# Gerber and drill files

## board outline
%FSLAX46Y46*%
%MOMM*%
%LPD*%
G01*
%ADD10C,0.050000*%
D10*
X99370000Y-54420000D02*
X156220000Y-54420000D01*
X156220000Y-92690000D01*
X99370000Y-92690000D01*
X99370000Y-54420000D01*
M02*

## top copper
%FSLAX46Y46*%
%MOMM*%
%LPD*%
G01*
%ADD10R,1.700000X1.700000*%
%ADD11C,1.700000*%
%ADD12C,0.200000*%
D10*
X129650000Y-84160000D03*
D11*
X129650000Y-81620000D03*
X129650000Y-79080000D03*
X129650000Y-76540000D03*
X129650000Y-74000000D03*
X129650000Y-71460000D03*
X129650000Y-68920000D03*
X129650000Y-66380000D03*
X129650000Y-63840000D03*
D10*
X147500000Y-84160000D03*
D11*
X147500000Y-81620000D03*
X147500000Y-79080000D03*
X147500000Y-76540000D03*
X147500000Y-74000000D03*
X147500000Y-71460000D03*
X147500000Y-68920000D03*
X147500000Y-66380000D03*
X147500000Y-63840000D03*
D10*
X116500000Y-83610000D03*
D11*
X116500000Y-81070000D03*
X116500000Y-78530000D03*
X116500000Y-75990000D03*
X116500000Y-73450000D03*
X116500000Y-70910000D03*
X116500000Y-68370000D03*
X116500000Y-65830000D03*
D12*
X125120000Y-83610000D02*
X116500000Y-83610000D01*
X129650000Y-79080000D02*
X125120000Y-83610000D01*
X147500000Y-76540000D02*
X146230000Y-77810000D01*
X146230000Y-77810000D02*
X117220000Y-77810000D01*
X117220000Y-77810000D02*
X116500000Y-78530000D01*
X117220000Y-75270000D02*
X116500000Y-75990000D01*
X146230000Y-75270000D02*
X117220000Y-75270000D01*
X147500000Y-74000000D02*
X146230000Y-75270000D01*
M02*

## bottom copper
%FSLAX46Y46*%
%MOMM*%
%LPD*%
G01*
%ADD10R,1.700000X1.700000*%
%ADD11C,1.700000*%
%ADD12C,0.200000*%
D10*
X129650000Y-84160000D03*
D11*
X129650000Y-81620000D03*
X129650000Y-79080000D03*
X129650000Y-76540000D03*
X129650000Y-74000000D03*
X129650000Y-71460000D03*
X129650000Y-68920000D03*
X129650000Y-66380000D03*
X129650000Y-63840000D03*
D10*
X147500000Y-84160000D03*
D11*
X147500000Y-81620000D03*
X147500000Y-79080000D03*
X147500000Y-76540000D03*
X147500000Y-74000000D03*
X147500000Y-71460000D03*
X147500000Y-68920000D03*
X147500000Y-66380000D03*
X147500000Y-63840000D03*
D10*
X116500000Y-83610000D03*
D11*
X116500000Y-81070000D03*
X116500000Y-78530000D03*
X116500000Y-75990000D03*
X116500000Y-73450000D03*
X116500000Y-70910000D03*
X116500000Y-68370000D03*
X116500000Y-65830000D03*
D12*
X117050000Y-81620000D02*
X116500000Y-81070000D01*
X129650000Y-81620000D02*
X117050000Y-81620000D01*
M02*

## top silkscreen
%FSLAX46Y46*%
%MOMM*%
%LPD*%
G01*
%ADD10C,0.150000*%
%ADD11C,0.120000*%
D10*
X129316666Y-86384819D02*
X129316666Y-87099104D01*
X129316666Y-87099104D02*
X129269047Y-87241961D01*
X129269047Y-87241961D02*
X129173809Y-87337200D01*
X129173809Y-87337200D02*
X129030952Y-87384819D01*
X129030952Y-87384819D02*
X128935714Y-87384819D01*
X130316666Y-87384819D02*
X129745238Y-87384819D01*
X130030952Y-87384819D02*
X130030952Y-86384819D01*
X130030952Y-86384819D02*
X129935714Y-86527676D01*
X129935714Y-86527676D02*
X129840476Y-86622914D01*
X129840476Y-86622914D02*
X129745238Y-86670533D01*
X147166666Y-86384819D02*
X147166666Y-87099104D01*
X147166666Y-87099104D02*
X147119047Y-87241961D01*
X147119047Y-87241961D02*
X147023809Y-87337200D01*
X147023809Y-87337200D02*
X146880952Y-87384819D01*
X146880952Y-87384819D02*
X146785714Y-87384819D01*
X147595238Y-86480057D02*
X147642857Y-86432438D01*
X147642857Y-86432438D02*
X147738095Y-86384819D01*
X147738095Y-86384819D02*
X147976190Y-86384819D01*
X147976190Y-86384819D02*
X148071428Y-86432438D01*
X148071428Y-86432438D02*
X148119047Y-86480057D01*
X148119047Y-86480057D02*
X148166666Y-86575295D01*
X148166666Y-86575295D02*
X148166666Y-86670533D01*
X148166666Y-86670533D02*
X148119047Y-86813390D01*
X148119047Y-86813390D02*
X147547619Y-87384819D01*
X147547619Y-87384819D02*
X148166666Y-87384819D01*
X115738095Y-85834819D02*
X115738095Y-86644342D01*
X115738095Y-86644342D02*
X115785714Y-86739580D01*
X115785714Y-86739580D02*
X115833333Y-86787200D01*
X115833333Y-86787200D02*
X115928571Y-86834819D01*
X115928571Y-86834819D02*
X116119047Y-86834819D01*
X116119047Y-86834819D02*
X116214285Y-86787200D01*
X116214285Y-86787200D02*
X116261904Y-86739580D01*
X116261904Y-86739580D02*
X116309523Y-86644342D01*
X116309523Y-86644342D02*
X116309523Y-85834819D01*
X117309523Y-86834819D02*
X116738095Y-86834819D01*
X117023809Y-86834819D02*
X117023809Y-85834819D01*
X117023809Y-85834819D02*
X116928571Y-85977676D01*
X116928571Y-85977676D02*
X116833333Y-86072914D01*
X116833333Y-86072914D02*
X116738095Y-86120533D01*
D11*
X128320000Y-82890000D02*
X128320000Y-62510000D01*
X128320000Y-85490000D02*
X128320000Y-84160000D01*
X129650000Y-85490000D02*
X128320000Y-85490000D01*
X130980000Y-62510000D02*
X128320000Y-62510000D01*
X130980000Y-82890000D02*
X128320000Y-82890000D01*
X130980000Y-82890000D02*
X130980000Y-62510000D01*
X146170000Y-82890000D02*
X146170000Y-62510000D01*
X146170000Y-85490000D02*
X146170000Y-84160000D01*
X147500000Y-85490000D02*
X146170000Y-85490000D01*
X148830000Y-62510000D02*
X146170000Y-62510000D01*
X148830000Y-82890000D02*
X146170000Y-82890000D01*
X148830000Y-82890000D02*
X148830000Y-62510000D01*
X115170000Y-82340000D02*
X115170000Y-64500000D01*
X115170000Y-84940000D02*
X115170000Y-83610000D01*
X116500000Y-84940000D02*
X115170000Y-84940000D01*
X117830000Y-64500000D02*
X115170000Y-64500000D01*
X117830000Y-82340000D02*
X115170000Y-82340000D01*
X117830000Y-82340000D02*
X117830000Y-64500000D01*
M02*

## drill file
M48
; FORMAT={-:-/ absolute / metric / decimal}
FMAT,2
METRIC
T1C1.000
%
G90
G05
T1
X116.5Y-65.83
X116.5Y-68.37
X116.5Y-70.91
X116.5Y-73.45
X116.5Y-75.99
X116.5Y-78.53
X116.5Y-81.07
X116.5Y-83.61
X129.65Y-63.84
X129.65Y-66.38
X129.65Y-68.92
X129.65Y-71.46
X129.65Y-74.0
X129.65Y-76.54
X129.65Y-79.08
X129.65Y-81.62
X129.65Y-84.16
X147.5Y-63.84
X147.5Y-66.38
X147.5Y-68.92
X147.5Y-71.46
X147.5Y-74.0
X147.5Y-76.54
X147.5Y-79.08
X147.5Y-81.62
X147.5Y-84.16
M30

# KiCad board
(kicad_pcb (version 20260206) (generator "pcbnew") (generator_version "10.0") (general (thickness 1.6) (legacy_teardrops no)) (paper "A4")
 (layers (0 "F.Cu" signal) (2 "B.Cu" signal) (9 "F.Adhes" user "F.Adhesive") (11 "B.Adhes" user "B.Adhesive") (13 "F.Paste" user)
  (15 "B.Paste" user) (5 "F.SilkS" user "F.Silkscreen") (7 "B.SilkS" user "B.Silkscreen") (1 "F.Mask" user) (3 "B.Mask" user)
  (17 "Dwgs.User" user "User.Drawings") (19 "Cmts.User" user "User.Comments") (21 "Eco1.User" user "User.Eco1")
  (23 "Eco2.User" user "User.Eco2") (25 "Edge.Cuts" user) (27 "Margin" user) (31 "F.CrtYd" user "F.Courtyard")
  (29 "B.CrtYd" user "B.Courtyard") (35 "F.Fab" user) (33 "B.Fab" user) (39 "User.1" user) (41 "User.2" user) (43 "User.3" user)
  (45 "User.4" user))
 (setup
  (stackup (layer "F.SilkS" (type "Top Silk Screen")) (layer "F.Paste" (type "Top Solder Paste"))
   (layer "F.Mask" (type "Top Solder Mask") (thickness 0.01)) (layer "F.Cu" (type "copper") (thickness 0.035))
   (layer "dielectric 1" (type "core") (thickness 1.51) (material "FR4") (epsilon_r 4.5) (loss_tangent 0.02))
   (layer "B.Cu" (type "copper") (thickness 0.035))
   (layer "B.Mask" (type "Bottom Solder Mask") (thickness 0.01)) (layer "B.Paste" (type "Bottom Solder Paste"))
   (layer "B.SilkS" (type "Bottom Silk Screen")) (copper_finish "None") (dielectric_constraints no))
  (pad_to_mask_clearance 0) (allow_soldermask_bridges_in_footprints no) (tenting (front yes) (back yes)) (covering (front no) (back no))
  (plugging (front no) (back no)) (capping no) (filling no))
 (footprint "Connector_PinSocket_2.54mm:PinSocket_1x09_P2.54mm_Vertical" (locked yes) (layer "F.Cu") (at 129.65 84.16 180)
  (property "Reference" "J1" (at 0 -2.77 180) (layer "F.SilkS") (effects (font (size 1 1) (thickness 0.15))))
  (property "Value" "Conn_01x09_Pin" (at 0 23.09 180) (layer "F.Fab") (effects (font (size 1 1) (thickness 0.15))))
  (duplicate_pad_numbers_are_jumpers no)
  (fp_line (start 1.33 1.27) (end 1.33 21.65) (stroke (width 0.12) (type solid)) (layer "F.SilkS"))
  (fp_line (start 1.33 -1.33) (end 1.33 0) (stroke (width 0.12) (type solid)) (layer "F.SilkS"))
  (fp_line (start 0 -1.33) (end 1.33 -1.33) (stroke (width 0.12) (type solid)) (layer "F.SilkS"))
  (fp_line (start -1.33 21.65) (end 1.33 21.65) (stroke (width 0.12) (type solid)) (layer "F.SilkS"))
  (fp_line (start -1.33 1.27) (end 1.33 1.27) (stroke (width 0.12) (type solid)) (layer "F.SilkS"))
  (fp_line (start -1.33 1.27) (end -1.33 21.65) (stroke (width 0.12) (type solid)) (layer "F.SilkS"))
  (pad "1" thru_hole rect (at 0 0 180) (size 1.7 1.7) (drill 1) (layers "*.Cu" "*.Mask") (remove_unused_layers no)
   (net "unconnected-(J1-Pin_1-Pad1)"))
  (pad "2" thru_hole circle (at 0 2.54 180) (size 1.7 1.7) (drill 1) (layers "*.Cu" "*.Mask") (remove_unused_layers no)
   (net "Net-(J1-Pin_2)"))
  (pad "3" thru_hole circle (at 0 5.08 180) (size 1.7 1.7) (drill 1) (layers "*.Cu" "*.Mask") (remove_unused_layers no)
   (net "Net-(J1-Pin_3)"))
  (pad "4" thru_hole circle (at 0 7.62 180) (size 1.7 1.7) (drill 1) (layers "*.Cu" "*.Mask") (remove_unused_layers no)
   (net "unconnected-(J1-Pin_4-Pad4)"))
  (pad "5" thru_hole circle (at 0 10.16 180) (size 1.7 1.7) (drill 1) (layers "*.Cu" "*.Mask") (remove_unused_layers no)
   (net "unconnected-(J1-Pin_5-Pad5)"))
  (pad "6" thru_hole circle (at 0 12.7 180) (size 1.7 1.7) (drill 1) (layers "*.Cu" "*.Mask") (remove_unused_layers no)
   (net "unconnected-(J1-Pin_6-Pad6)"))
  (pad "7" thru_hole circle (at 0 15.24 180) (size 1.7 1.7) (drill 1) (layers "*.Cu" "*.Mask") (remove_unused_layers no)
   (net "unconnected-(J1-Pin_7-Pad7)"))
  (pad "8" thru_hole circle (at 0 17.78 180) (size 1.7 1.7) (drill 1) (layers "*.Cu" "*.Mask") (remove_unused_layers no)
   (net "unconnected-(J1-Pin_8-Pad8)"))
  (pad "9" thru_hole circle (at 0 20.32 180) (size 1.7 1.7) (drill 1) (layers "*.Cu" "*.Mask") (remove_unused_layers no)
   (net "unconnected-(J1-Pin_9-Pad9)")))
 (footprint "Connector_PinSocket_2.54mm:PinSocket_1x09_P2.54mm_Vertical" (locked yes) (layer "F.Cu") (at 147.5 84.16 180)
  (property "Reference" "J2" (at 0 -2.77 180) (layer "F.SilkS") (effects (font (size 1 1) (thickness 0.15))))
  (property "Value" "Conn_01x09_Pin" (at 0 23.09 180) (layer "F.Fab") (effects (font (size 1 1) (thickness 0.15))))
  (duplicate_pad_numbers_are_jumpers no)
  (fp_line (start 1.33 1.27) (end 1.33 21.65) (stroke (width 0.12) (type solid)) (layer "F.SilkS"))
  (fp_line (start 1.33 -1.33) (end 1.33 0) (stroke (width 0.12) (type solid)) (layer "F.SilkS"))
  (fp_line (start 0 -1.33) (end 1.33 -1.33) (stroke (width 0.12) (type solid)) (layer "F.SilkS"))
  (fp_line (start -1.33 21.65) (end 1.33 21.65) (stroke (width 0.12) (type solid)) (layer "F.SilkS"))
  (fp_line (start -1.33 1.27) (end 1.33 1.27) (stroke (width 0.12) (type solid)) (layer "F.SilkS"))
  (fp_line (start -1.33 1.27) (end -1.33 21.65) (stroke (width 0.12) (type solid)) (layer "F.SilkS"))
  (pad "1" thru_hole rect (at 0 0 180) (size 1.7 1.7) (drill 1) (layers "*.Cu" "*.Mask") (remove_unused_layers no)
   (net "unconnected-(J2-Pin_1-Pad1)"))
  (pad "2" thru_hole circle (at 0 2.54 180) (size 1.7 1.7) (drill 1) (layers "*.Cu" "*.Mask") (remove_unused_layers no)
   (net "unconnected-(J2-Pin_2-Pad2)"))
  (pad "3" thru_hole circle (at 0 5.08 180) (size 1.7 1.7) (drill 1) (layers "*.Cu" "*.Mask") (remove_unused_layers no)
   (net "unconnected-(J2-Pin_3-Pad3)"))
  (pad "4" thru_hole circle (at 0 7.62 180) (size 1.7 1.7) (drill 1) (layers "*.Cu" "*.Mask") (remove_unused_layers no)
   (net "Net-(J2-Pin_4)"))
  (pad "5" thru_hole circle (at 0 10.16 180) (size 1.7 1.7) (drill 1) (layers "*.Cu" "*.Mask") (remove_unused_layers no)
   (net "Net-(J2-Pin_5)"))
  (pad "6" thru_hole circle (at 0 12.7 180) (size 1.7 1.7) (drill 1) (layers "*.Cu" "*.Mask") (remove_unused_layers no)
   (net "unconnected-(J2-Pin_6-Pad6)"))
  (pad "7" thru_hole circle (at 0 15.24 180) (size 1.7 1.7) (drill 1) (layers "*.Cu" "*.Mask") (remove_unused_layers no)
   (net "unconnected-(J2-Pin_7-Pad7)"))
  (pad "8" thru_hole circle (at 0 17.78 180) (size 1.7 1.7) (drill 1) (layers "*.Cu" "*.Mask") (remove_unused_layers no)
   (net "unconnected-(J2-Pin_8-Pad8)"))
  (pad "9" thru_hole circle (at 0 20.32 180) (size 1.7 1.7) (drill 1) (layers "*.Cu" "*.Mask") (remove_unused_layers no)
   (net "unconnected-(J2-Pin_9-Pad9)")))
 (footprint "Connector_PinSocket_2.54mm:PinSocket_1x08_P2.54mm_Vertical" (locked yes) (layer "F.Cu") (at 116.5 83.61 180)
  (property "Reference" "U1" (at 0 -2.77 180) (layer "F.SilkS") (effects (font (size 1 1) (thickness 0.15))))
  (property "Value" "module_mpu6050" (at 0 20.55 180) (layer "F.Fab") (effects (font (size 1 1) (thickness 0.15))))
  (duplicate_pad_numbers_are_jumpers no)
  (fp_line (start 1.33 1.27) (end 1.33 19.11) (stroke (width 0.12) (type solid)) (layer "F.SilkS"))
  (fp_line (start 1.33 -1.33) (end 1.33 0) (stroke (width 0.12) (type solid)) (layer "F.SilkS"))
  (fp_line (start 0 -1.33) (end 1.33 -1.33) (stroke (width 0.12) (type solid)) (layer "F.SilkS"))
  (fp_line (start -1.33 19.11) (end 1.33 19.11) (stroke (width 0.12) (type solid)) (layer "F.SilkS"))
  (fp_line (start -1.33 1.27) (end 1.33 1.27) (stroke (width 0.12) (type solid)) (layer "F.SilkS"))
  (fp_line (start -1.33 1.27) (end -1.33 19.11) (stroke (width 0.12) (type solid)) (layer "F.SilkS"))
  (pad "1" thru_hole rect (at 0 0 180) (size 1.7 1.7) (drill 1) (layers "*.Cu" "*.Mask") (remove_unused_layers no) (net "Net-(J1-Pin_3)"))
  (pad "2" thru_hole circle (at 0 2.54 180) (size 1.7 1.7) (drill 1) (layers "*.Cu" "*.Mask") (remove_unused_layers no)
   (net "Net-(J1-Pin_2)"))
  (pad "3" thru_hole circle (at 0 5.08 180) (size 1.7 1.7) (drill 1) (layers "*.Cu" "*.Mask") (remove_unused_layers no)
   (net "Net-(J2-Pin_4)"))
  (pad "4" thru_hole circle (at 0 7.62 180) (size 1.7 1.7) (drill 1) (layers "*.Cu" "*.Mask") (remove_unused_layers no)
   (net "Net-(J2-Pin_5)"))
  (pad "5" thru_hole circle (at 0 10.16 180) (size 1.7 1.7) (drill 1) (layers "*.Cu" "*.Mask") (remove_unused_layers no)
   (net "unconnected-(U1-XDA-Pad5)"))
  (pad "6" thru_hole circle (at 0 12.7 180) (size 1.7 1.7) (drill 1) (layers "*.Cu" "*.Mask") (remove_unused_layers no)
   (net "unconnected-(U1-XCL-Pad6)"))
  (pad "7" thru_hole circle (at 0 15.24 180) (size 1.7 1.7) (drill 1) (layers "*.Cu" "*.Mask") (remove_unused_layers no)
   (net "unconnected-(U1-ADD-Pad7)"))
  (pad "8" thru_hole circle (at 0 17.78 180) (size 1.7 1.7) (drill 1) (layers "*.Cu" "*.Mask") (remove_unused_layers no)
   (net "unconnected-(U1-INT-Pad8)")))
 (gr_rect (start 99.37 54.42) (end 156.22 92.69) (stroke (width 0.05) (type default)) (fill no) (locked yes) (layer "Edge.Cuts"))
 (segment (start 117.05 81.62) (end 116.5 81.07) (width 0.2) (layer "B.Cu") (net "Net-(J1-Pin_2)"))
 (segment (start 129.65 81.62) (end 117.05 81.62) (width 0.2) (layer "B.Cu") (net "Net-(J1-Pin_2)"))
 (segment (start 125.12 83.61) (end 116.5 83.61) (width 0.2) (layer "F.Cu") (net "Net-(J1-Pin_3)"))
 (segment (start 129.65 79.08) (end 125.12 83.61) (width 0.2) (layer "F.Cu") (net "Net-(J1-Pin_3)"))
 (segment (start 147.5 76.54) (end 146.23 77.81) (width 0.2) (layer "F.Cu") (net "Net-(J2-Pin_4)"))
 (segment (start 146.23 77.81) (end 117.22 77.81) (width 0.2) (layer "F.Cu") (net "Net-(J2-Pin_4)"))
 (segment (start 117.22 77.81) (end 116.5 78.53) (width 0.2) (layer "F.Cu") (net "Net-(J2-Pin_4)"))
 (segment (start 117.22 75.27) (end 116.5 75.99) (width 0.2) (layer "F.Cu") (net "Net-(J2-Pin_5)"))
 (segment (start 146.23 75.27) (end 117.22 75.27) (width 0.2) (layer "F.Cu") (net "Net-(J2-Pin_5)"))
 (segment (start 147.5 74) (end 146.23 75.27) (width 0.2) (layer "F.Cu") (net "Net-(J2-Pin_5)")))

